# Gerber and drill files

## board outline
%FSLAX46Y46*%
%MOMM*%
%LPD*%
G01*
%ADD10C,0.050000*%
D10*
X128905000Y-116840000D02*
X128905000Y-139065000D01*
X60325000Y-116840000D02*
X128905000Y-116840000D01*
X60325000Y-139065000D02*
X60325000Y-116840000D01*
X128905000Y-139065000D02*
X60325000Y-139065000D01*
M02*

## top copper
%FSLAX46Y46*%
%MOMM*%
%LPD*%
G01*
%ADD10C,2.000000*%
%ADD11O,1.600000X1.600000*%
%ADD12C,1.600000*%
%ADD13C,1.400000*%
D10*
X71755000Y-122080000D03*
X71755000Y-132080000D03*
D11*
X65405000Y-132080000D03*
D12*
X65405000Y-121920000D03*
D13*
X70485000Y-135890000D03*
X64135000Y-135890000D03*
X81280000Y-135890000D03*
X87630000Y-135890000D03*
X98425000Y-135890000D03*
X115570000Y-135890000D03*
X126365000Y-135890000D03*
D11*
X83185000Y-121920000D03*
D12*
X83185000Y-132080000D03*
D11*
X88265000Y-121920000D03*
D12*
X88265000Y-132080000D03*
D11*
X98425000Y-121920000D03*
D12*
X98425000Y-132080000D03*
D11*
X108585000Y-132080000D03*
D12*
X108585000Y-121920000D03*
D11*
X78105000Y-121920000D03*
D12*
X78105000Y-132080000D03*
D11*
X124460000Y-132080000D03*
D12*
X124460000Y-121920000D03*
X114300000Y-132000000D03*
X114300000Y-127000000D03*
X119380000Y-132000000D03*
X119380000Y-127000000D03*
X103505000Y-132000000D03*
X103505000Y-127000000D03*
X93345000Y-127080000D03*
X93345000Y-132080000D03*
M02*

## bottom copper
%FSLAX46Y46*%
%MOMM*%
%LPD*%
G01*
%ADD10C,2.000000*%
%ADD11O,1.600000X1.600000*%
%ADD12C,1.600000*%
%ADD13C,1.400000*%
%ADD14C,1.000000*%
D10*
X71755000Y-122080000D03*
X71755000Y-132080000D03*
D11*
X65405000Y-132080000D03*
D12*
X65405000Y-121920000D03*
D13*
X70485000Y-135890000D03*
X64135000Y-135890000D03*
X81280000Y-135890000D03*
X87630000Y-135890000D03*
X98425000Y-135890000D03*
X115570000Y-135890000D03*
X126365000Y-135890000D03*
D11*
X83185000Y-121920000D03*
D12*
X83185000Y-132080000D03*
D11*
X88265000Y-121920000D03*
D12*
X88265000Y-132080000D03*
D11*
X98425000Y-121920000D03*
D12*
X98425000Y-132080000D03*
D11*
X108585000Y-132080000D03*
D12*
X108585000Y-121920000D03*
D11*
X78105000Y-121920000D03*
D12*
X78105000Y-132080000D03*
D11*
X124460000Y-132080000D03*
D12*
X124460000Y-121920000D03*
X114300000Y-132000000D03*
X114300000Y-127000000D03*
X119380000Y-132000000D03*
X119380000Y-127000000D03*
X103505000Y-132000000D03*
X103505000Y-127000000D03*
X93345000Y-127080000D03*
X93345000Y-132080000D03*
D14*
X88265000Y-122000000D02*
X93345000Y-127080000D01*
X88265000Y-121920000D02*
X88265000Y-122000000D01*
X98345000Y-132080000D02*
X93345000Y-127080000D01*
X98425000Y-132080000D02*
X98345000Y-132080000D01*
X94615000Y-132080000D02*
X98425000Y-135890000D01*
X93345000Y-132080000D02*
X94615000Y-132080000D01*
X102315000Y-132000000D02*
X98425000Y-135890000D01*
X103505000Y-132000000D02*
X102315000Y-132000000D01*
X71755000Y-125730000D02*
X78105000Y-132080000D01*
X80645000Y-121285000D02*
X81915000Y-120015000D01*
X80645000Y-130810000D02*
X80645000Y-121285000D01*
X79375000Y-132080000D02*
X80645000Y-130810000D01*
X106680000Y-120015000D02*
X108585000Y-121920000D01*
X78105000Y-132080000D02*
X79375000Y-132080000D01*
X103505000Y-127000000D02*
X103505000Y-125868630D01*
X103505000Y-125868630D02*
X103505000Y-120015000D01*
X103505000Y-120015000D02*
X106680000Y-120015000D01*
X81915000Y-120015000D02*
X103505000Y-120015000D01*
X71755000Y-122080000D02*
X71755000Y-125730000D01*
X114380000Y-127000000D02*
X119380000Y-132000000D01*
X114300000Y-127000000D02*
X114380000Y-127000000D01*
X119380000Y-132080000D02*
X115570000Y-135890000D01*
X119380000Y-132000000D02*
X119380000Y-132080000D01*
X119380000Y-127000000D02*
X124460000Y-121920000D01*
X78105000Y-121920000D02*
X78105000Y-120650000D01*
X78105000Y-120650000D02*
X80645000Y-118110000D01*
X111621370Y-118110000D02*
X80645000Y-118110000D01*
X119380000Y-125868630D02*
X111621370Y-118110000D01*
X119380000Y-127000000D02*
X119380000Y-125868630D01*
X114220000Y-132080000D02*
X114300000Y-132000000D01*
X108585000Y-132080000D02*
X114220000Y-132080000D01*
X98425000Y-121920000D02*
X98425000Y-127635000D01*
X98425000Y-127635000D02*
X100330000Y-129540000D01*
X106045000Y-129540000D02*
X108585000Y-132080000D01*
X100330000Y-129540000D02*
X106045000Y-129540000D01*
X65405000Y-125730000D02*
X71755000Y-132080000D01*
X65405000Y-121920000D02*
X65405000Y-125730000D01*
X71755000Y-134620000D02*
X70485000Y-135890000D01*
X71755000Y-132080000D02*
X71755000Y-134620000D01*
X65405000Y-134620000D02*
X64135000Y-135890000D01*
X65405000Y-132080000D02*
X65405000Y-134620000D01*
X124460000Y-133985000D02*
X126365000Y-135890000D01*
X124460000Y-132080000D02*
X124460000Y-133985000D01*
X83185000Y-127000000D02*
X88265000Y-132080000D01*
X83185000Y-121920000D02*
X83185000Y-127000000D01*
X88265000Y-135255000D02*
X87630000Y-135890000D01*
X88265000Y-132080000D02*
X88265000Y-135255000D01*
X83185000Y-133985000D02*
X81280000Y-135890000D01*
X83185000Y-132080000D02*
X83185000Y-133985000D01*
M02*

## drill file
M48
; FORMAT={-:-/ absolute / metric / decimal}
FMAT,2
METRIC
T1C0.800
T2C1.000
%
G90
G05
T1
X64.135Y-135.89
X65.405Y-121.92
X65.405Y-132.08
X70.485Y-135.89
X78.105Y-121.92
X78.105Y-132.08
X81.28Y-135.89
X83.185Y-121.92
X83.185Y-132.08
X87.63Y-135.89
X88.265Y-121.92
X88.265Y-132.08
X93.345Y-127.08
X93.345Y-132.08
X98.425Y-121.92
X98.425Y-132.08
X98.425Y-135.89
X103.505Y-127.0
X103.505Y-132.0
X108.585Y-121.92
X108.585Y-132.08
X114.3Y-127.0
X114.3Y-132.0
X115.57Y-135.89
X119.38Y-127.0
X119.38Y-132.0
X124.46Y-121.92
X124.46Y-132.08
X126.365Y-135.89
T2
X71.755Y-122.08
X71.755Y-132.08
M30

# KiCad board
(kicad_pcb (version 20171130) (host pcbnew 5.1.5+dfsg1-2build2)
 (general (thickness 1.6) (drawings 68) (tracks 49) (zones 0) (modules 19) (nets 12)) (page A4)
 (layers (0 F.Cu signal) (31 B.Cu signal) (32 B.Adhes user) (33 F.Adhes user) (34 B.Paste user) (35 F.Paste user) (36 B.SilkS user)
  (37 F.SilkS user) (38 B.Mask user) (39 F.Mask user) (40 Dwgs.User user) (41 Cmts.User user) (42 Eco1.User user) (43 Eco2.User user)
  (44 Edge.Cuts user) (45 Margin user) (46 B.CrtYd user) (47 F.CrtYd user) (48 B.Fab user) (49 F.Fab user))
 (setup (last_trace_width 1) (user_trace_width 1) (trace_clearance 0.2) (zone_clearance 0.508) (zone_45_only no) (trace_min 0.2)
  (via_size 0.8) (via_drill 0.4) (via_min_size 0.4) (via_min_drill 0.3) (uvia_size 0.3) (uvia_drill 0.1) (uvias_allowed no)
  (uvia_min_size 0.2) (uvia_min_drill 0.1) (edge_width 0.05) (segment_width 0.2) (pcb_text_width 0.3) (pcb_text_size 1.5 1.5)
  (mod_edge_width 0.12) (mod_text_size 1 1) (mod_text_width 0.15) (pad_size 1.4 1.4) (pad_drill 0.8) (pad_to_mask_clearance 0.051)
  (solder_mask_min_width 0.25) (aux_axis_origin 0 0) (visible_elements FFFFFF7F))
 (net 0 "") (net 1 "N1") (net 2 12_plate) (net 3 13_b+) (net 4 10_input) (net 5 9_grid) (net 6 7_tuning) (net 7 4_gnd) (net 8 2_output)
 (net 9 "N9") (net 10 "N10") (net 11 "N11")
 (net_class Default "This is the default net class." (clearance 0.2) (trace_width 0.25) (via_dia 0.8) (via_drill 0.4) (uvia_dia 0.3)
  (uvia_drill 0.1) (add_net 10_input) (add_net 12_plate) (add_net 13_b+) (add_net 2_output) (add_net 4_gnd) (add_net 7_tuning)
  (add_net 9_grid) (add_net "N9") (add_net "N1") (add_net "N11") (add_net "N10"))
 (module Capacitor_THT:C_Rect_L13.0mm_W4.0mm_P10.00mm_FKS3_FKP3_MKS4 (layer F.Cu) (at 71.755 132.08 90)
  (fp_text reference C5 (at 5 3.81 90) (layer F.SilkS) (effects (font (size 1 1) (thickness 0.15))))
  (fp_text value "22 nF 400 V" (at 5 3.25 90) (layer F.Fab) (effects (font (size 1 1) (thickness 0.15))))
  (pad 2 thru_hole circle (at 10 0 90) (size 2 2) (drill 1) (layers *.Cu *.Mask) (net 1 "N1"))
  (pad 1 thru_hole circle (at 0 0 90) (size 2 2) (drill 1) (layers *.Cu *.Mask) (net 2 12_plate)))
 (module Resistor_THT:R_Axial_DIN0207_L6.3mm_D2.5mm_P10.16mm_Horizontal (layer F.Cu) (at 65.405 121.92 270)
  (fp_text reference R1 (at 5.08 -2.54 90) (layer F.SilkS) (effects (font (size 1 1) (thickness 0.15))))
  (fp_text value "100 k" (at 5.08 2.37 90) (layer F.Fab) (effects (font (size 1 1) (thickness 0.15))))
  (pad 2 thru_hole oval (at 10.16 0 270) (size 1.6 1.6) (drill 0.8) (layers *.Cu *.Mask) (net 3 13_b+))
  (pad 1 thru_hole circle (at 0 0 270) (size 1.6 1.6) (drill 0.8) (layers *.Cu *.Mask) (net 2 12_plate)))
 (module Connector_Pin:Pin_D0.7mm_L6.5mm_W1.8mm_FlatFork (layer F.Cu) (at 70.485 135.89)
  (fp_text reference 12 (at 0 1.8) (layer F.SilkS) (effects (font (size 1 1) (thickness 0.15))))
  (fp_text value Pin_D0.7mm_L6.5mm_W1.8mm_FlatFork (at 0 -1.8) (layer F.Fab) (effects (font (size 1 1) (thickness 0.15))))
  (pad 12 thru_hole circle (at 0 0) (size 1.4 1.4) (drill 0.8) (layers *.Cu *.Mask) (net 2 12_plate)))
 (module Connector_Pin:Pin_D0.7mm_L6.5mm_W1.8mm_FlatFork (layer F.Cu) (at 64.135 135.89)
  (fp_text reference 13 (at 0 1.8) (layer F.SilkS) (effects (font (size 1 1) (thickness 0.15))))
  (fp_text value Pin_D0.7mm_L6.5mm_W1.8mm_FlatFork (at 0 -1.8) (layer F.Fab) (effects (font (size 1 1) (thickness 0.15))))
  (pad 13 thru_hole circle (at 0 0) (size 1.4 1.4) (drill 0.8) (layers *.Cu *.Mask) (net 3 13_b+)))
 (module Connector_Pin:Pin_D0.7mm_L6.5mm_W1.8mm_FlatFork (layer F.Cu) (at 81.28 135.89)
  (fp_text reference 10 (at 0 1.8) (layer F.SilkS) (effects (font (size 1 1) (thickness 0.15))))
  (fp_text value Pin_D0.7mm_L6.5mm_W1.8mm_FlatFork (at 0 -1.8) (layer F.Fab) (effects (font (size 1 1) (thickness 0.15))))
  (pad 10 thru_hole circle (at 0 0) (size 1.4 1.4) (drill 0.8) (layers *.Cu *.Mask) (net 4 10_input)))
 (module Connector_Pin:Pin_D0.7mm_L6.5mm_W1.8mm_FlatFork (layer F.Cu) (at 87.63 135.89)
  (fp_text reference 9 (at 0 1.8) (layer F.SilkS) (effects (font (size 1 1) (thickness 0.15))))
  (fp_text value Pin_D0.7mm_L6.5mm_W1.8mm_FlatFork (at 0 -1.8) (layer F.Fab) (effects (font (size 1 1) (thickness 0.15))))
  (pad 9 thru_hole circle (at 0 0) (size 1.4 1.4) (drill 0.8) (layers *.Cu *.Mask) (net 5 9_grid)))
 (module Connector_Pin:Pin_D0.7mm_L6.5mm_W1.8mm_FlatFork (layer F.Cu) (at 98.425 135.89)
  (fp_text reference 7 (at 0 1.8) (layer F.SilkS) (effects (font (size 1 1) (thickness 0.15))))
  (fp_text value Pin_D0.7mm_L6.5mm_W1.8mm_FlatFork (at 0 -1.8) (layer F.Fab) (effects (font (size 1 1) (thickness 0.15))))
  (pad 7 thru_hole circle (at 0 0) (size 1.4 1.4) (drill 0.8) (layers *.Cu *.Mask) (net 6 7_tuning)))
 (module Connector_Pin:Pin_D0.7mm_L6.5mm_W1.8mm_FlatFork (layer F.Cu) (at 115.57 135.89)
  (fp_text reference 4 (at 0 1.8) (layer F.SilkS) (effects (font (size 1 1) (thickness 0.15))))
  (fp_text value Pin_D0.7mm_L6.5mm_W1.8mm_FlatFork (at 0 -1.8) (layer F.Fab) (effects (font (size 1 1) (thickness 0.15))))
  (pad 4 thru_hole circle (at 0 0) (size 1.4 1.4) (drill 0.8) (layers *.Cu *.Mask) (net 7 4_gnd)))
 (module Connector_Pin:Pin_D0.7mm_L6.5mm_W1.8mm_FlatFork (layer F.Cu) (at 126.365 135.89)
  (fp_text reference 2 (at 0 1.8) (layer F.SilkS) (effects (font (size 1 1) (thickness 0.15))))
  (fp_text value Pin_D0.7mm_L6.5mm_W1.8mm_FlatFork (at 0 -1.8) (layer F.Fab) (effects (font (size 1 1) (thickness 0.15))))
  (pad 2 thru_hole circle (at 0 0) (size 1.4 1.4) (drill 0.8) (layers *.Cu *.Mask) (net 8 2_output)))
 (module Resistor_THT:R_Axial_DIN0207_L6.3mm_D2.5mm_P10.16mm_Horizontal (layer F.Cu) (at 83.185 132.08 90)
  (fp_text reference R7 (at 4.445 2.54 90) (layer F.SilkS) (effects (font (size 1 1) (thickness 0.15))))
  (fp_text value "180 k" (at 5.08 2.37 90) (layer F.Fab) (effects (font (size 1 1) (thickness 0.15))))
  (pad 2 thru_hole oval (at 10.16 0 90) (size 1.6 1.6) (drill 0.8) (layers *.Cu *.Mask) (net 5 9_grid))
  (pad 1 thru_hole circle (at 0 0 90) (size 1.6 1.6) (drill 0.8) (layers *.Cu *.Mask) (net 4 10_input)))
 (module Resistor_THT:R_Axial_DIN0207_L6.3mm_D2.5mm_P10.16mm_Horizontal (layer F.Cu) (at 88.265 132.08 90)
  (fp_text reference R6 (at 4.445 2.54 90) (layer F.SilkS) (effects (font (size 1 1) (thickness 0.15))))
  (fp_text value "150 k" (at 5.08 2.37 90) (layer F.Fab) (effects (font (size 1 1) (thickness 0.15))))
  (pad 2 thru_hole oval (at 10.16 0 90) (size 1.6 1.6) (drill 0.8) (layers *.Cu *.Mask) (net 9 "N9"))
  (pad 1 thru_hole circle (at 0 0 90) (size 1.6 1.6) (drill 0.8) (layers *.Cu *.Mask) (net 5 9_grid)))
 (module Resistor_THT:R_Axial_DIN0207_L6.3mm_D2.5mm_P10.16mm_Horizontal (layer F.Cu) (at 98.425 132.08 90)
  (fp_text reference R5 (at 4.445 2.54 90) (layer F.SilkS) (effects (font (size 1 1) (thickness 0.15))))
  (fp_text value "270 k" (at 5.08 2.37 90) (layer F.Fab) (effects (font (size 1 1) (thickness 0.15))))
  (pad 2 thru_hole oval (at 10.16 0 90) (size 1.6 1.6) (drill 0.8) (layers *.Cu *.Mask) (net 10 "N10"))
  (pad 1 thru_hole circle (at 0 0 90) (size 1.6 1.6) (drill 0.8) (layers *.Cu *.Mask) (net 9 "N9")))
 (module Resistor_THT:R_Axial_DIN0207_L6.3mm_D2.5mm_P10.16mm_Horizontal (layer F.Cu) (at 108.585 121.92 270)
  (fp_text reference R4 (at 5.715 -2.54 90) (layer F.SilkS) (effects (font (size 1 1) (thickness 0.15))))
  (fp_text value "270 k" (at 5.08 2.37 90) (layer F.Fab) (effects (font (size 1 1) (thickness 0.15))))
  (pad 2 thru_hole oval (at 10.16 0 270) (size 1.6 1.6) (drill 0.8) (layers *.Cu *.Mask) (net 10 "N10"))
  (pad 1 thru_hole circle (at 0 0 270) (size 1.6 1.6) (drill 0.8) (layers *.Cu *.Mask) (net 1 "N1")))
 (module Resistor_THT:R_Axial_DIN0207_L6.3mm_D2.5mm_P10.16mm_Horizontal (layer F.Cu) (at 78.105 132.08 90)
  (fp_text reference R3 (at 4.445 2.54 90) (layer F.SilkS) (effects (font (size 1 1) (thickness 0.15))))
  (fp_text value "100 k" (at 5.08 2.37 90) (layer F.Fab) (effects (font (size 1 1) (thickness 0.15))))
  (pad 2 thru_hole oval (at 10.16 0 90) (size 1.6 1.6) (drill 0.8) (layers *.Cu *.Mask) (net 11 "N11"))
  (pad 1 thru_hole circle (at 0 0 90) (size 1.6 1.6) (drill 0.8) (layers *.Cu *.Mask) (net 1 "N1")))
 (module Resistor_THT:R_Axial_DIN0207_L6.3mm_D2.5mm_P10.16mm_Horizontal (layer F.Cu) (at 124.46 121.92 270)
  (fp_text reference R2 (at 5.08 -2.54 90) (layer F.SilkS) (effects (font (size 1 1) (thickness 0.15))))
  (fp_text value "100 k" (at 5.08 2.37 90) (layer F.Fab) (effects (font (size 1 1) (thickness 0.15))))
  (pad 2 thru_hole oval (at 10.16 0 270) (size 1.6 1.6) (drill 0.8) (layers *.Cu *.Mask) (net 8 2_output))
  (pad 1 thru_hole circle (at 0 0 270) (size 1.6 1.6) (drill 0.8) (layers *.Cu *.Mask) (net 11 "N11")))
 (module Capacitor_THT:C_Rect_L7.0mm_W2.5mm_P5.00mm (layer F.Cu) (at 114.3 127 270)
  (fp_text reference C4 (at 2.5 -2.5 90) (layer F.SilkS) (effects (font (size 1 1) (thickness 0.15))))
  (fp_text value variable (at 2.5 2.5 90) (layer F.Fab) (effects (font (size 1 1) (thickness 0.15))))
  (pad 2 thru_hole circle (at 5 0 270) (size 1.6 1.6) (drill 0.8) (layers *.Cu *.Mask) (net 10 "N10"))
  (pad 1 thru_hole circle (at 0 0 270) (size 1.6 1.6) (drill 0.8) (layers *.Cu *.Mask) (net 7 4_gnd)))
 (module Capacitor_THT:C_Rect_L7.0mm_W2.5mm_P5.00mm (layer F.Cu) (at 119.38 127 270)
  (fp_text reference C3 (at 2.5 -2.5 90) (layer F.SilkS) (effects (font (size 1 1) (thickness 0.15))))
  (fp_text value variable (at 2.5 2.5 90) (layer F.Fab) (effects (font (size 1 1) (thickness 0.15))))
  (pad 2 thru_hole circle (at 5 0 270) (size 1.6 1.6) (drill 0.8) (layers *.Cu *.Mask) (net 7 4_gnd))
  (pad 1 thru_hole circle (at 0 0 270) (size 1.6 1.6) (drill 0.8) (layers *.Cu *.Mask) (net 11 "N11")))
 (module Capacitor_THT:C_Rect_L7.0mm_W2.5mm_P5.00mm (layer F.Cu) (at 103.505 127 270)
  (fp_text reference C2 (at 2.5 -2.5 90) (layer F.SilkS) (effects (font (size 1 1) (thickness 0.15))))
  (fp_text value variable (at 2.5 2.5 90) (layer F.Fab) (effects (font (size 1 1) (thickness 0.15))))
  (pad 2 thru_hole circle (at 5 0 270) (size 1.6 1.6) (drill 0.8) (layers *.Cu *.Mask) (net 6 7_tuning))
  (pad 1 thru_hole circle (at 0 0 270) (size 1.6 1.6) (drill 0.8) (layers *.Cu *.Mask) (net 1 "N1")))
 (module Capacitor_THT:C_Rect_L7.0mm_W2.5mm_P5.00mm (layer F.Cu) (at 93.345 132.08 90)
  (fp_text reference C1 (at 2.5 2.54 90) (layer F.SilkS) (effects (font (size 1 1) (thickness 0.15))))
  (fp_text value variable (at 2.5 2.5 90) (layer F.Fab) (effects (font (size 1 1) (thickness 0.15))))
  (pad 2 thru_hole circle (at 5 0 90) (size 1.6 1.6) (drill 0.8) (layers *.Cu *.Mask) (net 9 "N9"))
  (pad 1 thru_hole circle (at 0 0 90) (size 1.6 1.6) (drill 0.8) (layers *.Cu *.Mask) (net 6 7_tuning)))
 (gr_line (start 128.905 116.84) (end 128.905 139.065) (layer Edge.Cuts) (width 0.05))
 (gr_line (start 60.325 116.84) (end 128.905 116.84) (layer Edge.Cuts) (width 0.05))
 (gr_line (start 60.325 139.065) (end 60.325 116.84) (layer Edge.Cuts) (width 0.05))
 (gr_line (start 128.905 139.065) (end 60.325 139.065) (layer Edge.Cuts) (width 0.05))
 (segment (start 88.265 122) (end 93.345 127.08) (width 1) (layer B.Cu) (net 9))
 (segment (start 88.265 121.92) (end 88.265 122) (width 1) (layer B.Cu) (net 9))
 (segment (start 98.345 132.08) (end 93.345 127.08) (width 1) (layer B.Cu) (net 9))
 (segment (start 98.425 132.08) (end 98.345 132.08) (width 1) (layer B.Cu) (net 9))
 (segment (start 94.615 132.08) (end 98.425 135.89) (width 1) (layer B.Cu) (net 6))
 (segment (start 93.345 132.08) (end 94.615 132.08) (width 1) (layer B.Cu) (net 6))
 (segment (start 102.315 132) (end 98.425 135.89) (width 1) (layer B.Cu) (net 6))
 (segment (start 103.505 132) (end 102.315 132) (width 1) (layer B.Cu) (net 6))
 (segment (start 71.755 125.73) (end 78.105 132.08) (width 1) (layer B.Cu) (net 1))
 (segment (start 80.645 121.285) (end 81.915 120.015) (width 1) (layer B.Cu) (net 1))
 (segment (start 80.645 130.81) (end 80.645 121.285) (width 1) (layer B.Cu) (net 1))
 (segment (start 79.375 132.08) (end 80.645 130.81) (width 1) (layer B.Cu) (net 1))
 (segment (start 106.68 120.015) (end 108.585 121.92) (width 1) (layer B.Cu) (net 1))
 (segment (start 78.105 132.08) (end 79.375 132.08) (width 1) (layer B.Cu) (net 1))
 (segment (start 103.505 127) (end 103.505 125.86863) (width 1) (layer B.Cu) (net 1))
 (segment (start 103.505 125.86863) (end 103.505 120.015) (width 1) (layer B.Cu) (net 1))
 (segment (start 103.505 120.015) (end 106.68 120.015) (width 1) (layer B.Cu) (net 1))
 (segment (start 81.915 120.015) (end 103.505 120.015) (width 1) (layer B.Cu) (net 1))
 (segment (start 71.755 122.08) (end 71.755 125.73) (width 1) (layer B.Cu) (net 1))
 (segment (start 114.38 127) (end 119.38 132) (width 1) (layer B.Cu) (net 7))
 (segment (start 114.3 127) (end 114.38 127) (width 1) (layer B.Cu) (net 7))
 (segment (start 119.38 132.08) (end 115.57 135.89) (width 1) (layer B.Cu) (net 7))
 (segment (start 119.38 132) (end 119.38 132.08) (width 1) (layer B.Cu) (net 7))
 (segment (start 119.38 127) (end 124.46 121.92) (width 1) (layer B.Cu) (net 11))
 (segment (start 78.105 121.92) (end 78.105 120.65) (width 1) (layer B.Cu) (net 11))
 (segment (start 78.105 120.65) (end 80.645 118.11) (width 1) (layer B.Cu) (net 11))
 (segment (start 111.62137 118.11) (end 80.645 118.11) (width 1) (layer B.Cu) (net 11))
 (segment (start 119.38 125.86863) (end 111.62137 118.11) (width 1) (layer B.Cu) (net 11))
 (segment (start 119.38 127) (end 119.38 125.86863) (width 1) (layer B.Cu) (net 11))
 (segment (start 114.22 132.08) (end 114.3 132) (width 1) (layer B.Cu) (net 10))
 (segment (start 108.585 132.08) (end 114.22 132.08) (width 1) (layer B.Cu) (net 10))
 (segment (start 98.425 121.92) (end 98.425 127.635) (width 1) (layer B.Cu) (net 10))
 (segment (start 98.425 127.635) (end 100.33 129.54) (width 1) (layer B.Cu) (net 10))
 (segment (start 106.045 129.54) (end 108.585 132.08) (width 1) (layer B.Cu) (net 10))
 (segment (start 100.33 129.54) (end 106.045 129.54) (width 1) (layer B.Cu) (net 10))
 (segment (start 65.405 125.73) (end 71.755 132.08) (width 1) (layer B.Cu) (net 2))
 (segment (start 65.405 121.92) (end 65.405 125.73) (width 1) (layer B.Cu) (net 2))
 (segment (start 71.755 134.62) (end 70.485 135.89) (width 1) (layer B.Cu) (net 2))
 (segment (start 71.755 132.08) (end 71.755 134.62) (width 1) (layer B.Cu) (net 2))
 (segment (start 65.405 134.62) (end 64.135 135.89) (width 1) (layer B.Cu) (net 3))
 (segment (start 65.405 132.08) (end 65.405 134.62) (width 1) (layer B.Cu) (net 3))
 (segment (start 124.46 133.985) (end 126.365 135.89) (width 1) (layer B.Cu) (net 8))
 (segment (start 124.46 132.08) (end 124.46 133.985) (width 1) (layer B.Cu) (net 8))
 (segment (start 83.185 127) (end 88.265 132.08) (width 1) (layer B.Cu) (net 5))
 (segment (start 83.185 121.92) (end 83.185 127) (width 1) (layer B.Cu) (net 5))
 (segment (start 88.265 135.255) (end 87.63 135.89) (width 1) (layer B.Cu) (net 5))
 (segment (start 88.265 132.08) (end 88.265 135.255) (width 1) (layer B.Cu) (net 5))
 (segment (start 83.185 133.985) (end 81.28 135.89) (width 1) (layer B.Cu) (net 4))
 (segment (start 83.185 132.08) (end 83.185 133.985) (width 1) (layer B.Cu) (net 4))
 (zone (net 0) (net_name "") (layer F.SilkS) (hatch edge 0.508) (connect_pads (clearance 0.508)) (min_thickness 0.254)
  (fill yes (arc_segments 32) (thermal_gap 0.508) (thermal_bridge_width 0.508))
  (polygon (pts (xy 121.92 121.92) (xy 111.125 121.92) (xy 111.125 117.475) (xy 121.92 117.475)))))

